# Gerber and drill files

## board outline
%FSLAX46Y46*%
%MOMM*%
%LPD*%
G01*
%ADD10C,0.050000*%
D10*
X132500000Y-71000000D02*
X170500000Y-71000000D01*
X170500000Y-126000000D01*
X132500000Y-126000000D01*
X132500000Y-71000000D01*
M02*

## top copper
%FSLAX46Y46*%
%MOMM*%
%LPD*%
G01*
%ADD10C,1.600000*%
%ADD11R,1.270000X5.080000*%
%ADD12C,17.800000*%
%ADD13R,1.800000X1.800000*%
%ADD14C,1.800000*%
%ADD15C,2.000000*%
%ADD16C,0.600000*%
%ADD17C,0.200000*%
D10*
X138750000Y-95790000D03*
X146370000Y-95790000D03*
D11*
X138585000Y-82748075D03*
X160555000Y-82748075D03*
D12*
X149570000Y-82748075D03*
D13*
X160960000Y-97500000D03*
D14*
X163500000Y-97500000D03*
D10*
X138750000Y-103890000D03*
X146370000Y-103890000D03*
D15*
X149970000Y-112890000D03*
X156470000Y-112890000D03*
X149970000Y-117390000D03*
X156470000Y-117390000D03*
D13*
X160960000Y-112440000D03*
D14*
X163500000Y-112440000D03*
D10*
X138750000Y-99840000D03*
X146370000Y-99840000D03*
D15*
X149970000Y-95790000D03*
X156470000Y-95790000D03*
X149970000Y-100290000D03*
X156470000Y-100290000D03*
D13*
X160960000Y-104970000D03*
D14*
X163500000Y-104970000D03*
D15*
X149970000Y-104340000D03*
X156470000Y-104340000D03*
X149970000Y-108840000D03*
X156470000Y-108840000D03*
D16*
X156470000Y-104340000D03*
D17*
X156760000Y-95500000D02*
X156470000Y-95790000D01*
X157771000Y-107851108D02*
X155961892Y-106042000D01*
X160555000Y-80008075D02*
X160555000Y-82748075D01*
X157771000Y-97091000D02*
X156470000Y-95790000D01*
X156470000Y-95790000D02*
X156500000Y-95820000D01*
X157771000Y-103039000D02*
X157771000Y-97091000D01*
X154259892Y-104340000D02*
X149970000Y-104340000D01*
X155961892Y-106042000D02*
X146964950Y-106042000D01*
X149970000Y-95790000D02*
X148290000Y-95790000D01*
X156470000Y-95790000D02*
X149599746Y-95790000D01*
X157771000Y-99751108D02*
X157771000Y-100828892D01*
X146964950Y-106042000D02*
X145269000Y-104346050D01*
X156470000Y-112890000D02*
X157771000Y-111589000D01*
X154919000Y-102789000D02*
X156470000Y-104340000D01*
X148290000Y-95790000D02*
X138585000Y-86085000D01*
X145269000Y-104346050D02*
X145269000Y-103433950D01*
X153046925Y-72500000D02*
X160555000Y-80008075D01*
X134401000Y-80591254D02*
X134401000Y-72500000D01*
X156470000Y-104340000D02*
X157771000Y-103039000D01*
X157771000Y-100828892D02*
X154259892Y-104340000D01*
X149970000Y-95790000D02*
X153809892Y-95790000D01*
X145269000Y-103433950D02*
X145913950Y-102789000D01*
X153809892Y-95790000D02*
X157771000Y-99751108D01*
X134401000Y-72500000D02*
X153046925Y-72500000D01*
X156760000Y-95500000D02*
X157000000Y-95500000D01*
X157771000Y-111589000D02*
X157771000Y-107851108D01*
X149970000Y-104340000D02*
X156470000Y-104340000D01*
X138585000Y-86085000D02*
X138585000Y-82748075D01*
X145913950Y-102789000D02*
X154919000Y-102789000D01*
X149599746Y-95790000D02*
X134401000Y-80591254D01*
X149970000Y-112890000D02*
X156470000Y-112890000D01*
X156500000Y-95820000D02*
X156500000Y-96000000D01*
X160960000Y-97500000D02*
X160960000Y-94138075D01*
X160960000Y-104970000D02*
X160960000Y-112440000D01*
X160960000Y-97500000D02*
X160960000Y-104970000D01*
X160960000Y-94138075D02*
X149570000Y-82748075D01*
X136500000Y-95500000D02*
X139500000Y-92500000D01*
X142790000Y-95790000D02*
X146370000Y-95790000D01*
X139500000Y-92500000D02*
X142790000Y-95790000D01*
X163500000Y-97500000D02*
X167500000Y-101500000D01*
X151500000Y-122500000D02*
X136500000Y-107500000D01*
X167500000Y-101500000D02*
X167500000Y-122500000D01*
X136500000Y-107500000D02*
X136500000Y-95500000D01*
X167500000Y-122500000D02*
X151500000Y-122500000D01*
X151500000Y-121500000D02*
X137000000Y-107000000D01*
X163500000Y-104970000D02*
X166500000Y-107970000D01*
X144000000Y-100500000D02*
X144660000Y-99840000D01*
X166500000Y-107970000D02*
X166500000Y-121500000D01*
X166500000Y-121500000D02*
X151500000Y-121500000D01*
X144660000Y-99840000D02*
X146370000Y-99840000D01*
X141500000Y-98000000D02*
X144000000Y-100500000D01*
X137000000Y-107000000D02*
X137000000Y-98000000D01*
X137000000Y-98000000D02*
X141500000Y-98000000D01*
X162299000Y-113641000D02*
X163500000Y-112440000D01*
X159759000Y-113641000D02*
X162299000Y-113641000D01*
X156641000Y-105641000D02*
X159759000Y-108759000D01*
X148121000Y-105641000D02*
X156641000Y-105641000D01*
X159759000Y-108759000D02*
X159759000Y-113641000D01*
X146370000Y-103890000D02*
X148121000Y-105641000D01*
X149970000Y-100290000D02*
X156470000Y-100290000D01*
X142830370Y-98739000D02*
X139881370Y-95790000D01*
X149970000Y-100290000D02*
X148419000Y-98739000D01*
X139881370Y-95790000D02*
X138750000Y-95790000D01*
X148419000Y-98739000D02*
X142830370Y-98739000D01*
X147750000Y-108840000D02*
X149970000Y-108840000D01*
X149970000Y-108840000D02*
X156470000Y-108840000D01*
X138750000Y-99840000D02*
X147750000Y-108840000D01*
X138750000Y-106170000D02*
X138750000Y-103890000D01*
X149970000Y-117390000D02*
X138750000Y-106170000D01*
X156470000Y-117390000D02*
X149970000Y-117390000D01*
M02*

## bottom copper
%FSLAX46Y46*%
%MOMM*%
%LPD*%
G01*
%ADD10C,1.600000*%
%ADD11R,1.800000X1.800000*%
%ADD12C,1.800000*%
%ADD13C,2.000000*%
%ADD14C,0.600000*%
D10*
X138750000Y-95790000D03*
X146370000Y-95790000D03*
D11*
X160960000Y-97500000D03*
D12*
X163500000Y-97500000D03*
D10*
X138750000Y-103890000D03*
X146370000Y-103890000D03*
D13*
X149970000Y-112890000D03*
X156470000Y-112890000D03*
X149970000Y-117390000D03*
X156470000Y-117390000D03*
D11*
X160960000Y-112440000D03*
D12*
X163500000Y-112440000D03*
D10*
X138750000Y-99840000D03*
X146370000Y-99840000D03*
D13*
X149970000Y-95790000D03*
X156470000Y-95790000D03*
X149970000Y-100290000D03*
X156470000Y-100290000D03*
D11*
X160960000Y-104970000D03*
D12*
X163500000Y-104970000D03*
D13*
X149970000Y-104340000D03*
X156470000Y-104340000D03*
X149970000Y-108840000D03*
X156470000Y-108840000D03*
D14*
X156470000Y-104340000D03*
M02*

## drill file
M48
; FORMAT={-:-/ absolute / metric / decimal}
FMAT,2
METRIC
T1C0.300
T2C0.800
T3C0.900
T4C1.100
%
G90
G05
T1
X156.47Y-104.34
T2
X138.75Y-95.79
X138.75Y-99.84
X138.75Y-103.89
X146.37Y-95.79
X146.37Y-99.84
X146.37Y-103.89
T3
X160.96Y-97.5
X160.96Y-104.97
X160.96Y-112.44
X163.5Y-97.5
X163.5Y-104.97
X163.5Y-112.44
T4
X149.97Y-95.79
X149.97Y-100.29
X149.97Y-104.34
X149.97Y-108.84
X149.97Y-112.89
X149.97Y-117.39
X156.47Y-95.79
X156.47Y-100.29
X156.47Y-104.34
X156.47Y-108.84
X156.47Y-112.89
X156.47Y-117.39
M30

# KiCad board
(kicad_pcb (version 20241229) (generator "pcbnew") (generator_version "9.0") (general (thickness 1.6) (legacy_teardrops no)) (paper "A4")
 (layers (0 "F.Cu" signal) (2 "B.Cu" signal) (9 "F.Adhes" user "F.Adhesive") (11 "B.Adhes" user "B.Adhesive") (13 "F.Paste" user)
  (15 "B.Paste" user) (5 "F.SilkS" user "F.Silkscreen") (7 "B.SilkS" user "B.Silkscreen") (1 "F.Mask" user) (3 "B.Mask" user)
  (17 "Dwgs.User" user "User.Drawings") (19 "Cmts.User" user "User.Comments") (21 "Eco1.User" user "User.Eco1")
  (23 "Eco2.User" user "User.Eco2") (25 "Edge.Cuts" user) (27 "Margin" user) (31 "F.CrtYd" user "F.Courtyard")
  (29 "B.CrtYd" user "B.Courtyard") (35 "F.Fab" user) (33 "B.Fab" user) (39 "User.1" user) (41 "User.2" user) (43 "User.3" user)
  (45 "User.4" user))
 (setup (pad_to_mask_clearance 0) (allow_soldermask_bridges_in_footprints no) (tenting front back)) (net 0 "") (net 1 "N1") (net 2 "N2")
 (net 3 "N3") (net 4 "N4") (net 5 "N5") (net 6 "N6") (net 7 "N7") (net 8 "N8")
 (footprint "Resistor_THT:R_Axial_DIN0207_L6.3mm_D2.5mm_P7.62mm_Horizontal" (layer "F.Cu") (at 138.75 95.79)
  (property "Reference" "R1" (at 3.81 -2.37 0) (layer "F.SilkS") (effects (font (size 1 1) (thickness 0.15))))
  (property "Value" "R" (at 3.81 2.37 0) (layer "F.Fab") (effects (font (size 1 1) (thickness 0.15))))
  (pad "1" thru_hole circle (at 0 0) (size 1.6 1.6) (drill 0.8) (layers "*.Cu" "*.Mask") (remove_unused_layers no) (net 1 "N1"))
  (pad "2" thru_hole circle (at 7.62 0) (size 1.6 1.6) (drill 0.8) (layers "*.Cu" "*.Mask") (remove_unused_layers no) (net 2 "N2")))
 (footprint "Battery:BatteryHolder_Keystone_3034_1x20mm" (layer "F.Cu") (at 149.57 82.748075)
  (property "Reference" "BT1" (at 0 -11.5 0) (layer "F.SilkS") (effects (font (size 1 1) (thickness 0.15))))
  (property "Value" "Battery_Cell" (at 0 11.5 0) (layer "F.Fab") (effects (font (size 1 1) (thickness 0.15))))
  (pad "1" smd rect (at -10.985 0) (size 1.27 5.08) (layers "F.Cu" "F.Mask" "F.Paste") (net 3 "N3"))
  (pad "1" smd rect (at 10.985 0) (size 1.27 5.08) (layers "F.Cu" "F.Mask" "F.Paste") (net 3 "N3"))
  (pad "2" smd circle (at 0 0) (size 17.8 17.8) (layers "F.Cu" "F.Mask") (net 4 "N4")))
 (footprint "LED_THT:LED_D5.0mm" (layer "F.Cu") (at 160.96 97.5)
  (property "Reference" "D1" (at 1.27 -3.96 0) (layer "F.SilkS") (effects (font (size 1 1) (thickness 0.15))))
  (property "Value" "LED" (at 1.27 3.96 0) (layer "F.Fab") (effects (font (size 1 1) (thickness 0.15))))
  (pad "1" thru_hole rect (at 0 0) (size 1.8 1.8) (drill 0.9) (layers "*.Cu" "*.Mask") (remove_unused_layers no) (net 4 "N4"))
  (pad "2" thru_hole circle (at 2.54 0) (size 1.8 1.8) (drill 0.9) (layers "*.Cu" "*.Mask") (remove_unused_layers no) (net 2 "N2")))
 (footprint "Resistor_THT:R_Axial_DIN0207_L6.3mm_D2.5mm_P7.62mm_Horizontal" (layer "F.Cu") (at 138.75 103.89)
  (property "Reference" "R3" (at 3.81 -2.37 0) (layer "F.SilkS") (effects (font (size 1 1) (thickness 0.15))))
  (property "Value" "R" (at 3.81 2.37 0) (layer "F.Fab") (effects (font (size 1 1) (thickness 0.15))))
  (pad "1" thru_hole circle (at 0 0) (size 1.6 1.6) (drill 0.8) (layers "*.Cu" "*.Mask") (remove_unused_layers no) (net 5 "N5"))
  (pad "2" thru_hole circle (at 7.62 0) (size 1.6 1.6) (drill 0.8) (layers "*.Cu" "*.Mask") (remove_unused_layers no) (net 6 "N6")))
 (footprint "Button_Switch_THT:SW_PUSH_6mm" (layer "F.Cu") (at 149.97 112.89)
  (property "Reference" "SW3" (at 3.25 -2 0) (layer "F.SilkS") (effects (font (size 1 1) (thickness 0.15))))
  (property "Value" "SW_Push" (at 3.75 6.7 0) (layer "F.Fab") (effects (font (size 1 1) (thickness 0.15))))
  (pad "1" thru_hole circle (at 0 0 90) (size 2 2) (drill 1.1) (layers "*.Cu" "*.Mask") (remove_unused_layers no) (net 3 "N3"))
  (pad "1" thru_hole circle (at 6.5 0 90) (size 2 2) (drill 1.1) (layers "*.Cu" "*.Mask") (remove_unused_layers no) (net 3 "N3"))
  (pad "2" thru_hole circle (at 0 4.5 90) (size 2 2) (drill 1.1) (layers "*.Cu" "*.Mask") (remove_unused_layers no) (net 5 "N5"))
  (pad "2" thru_hole circle (at 6.5 4.5 90) (size 2 2) (drill 1.1) (layers "*.Cu" "*.Mask") (remove_unused_layers no) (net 5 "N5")))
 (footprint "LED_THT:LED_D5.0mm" (layer "F.Cu") (at 160.96 112.44)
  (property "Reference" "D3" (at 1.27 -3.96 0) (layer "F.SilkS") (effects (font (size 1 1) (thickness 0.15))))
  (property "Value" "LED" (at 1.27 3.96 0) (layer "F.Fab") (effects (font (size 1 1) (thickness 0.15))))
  (pad "1" thru_hole rect (at 0 0) (size 1.8 1.8) (drill 0.9) (layers "*.Cu" "*.Mask") (remove_unused_layers no) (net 4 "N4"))
  (pad "2" thru_hole circle (at 2.54 0) (size 1.8 1.8) (drill 0.9) (layers "*.Cu" "*.Mask") (remove_unused_layers no) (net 6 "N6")))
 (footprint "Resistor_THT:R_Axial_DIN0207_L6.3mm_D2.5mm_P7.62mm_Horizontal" (layer "F.Cu") (at 138.75 99.84)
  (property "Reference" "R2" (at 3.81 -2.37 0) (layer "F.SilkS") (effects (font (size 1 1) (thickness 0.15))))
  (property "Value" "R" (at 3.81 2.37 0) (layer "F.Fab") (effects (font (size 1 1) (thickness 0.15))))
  (pad "1" thru_hole circle (at 0 0) (size 1.6 1.6) (drill 0.8) (layers "*.Cu" "*.Mask") (remove_unused_layers no) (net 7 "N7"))
  (pad "2" thru_hole circle (at 7.62 0) (size 1.6 1.6) (drill 0.8) (layers "*.Cu" "*.Mask") (remove_unused_layers no) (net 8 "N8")))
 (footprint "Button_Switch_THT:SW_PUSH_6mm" (layer "F.Cu") (at 149.97 95.79)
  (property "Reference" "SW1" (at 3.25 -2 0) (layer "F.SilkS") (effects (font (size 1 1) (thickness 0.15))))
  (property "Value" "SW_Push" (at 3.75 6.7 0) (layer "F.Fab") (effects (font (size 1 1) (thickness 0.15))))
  (pad "1" thru_hole circle (at 0 0 90) (size 2 2) (drill 1.1) (layers "*.Cu" "*.Mask") (remove_unused_layers no) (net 3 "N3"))
  (pad "1" thru_hole circle (at 6.5 0 90) (size 2 2) (drill 1.1) (layers "*.Cu" "*.Mask") (remove_unused_layers no) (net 3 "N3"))
  (pad "2" thru_hole circle (at 0 4.5 90) (size 2 2) (drill 1.1) (layers "*.Cu" "*.Mask") (remove_unused_layers no) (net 1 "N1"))
  (pad "2" thru_hole circle (at 6.5 4.5 90) (size 2 2) (drill 1.1) (layers "*.Cu" "*.Mask") (remove_unused_layers no) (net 1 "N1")))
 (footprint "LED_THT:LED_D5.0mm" (layer "F.Cu") (at 160.96 104.97)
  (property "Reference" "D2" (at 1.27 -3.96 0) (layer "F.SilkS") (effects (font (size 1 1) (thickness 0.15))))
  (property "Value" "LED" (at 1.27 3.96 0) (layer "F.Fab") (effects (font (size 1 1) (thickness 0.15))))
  (pad "1" thru_hole rect (at 0 0) (size 1.8 1.8) (drill 0.9) (layers "*.Cu" "*.Mask") (remove_unused_layers no) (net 4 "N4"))
  (pad "2" thru_hole circle (at 2.54 0) (size 1.8 1.8) (drill 0.9) (layers "*.Cu" "*.Mask") (remove_unused_layers no) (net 8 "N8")))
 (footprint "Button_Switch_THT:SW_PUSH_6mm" (layer "F.Cu") (at 149.97 104.34)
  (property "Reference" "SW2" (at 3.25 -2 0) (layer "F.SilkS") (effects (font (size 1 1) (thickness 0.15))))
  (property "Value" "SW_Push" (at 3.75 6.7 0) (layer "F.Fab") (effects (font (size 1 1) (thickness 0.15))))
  (pad "1" thru_hole circle (at 0 0 90) (size 2 2) (drill 1.1) (layers "*.Cu" "*.Mask") (remove_unused_layers no) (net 3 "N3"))
  (pad "1" thru_hole circle (at 6.5 0 90) (size 2 2) (drill 1.1) (layers "*.Cu" "*.Mask") (remove_unused_layers no) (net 3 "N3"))
  (pad "2" thru_hole circle (at 0 4.5 90) (size 2 2) (drill 1.1) (layers "*.Cu" "*.Mask") (remove_unused_layers no) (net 7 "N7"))
  (pad "2" thru_hole circle (at 6.5 4.5 90) (size 2 2) (drill 1.1) (layers "*.Cu" "*.Mask") (remove_unused_layers no) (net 7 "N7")))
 (gr_rect (start 132.5 71) (end 170.5 126) (stroke (width 0.05) (type default)) (fill no) (layer "Edge.Cuts"))
 (segment (start 156.76 95.5) (end 156.47 95.79) (width 0.2) (layer "F.Cu") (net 3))
 (segment (start 157.771 107.851108) (end 155.961892 106.042) (width 0.2) (layer "F.Cu") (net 3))
 (segment (start 160.555 80.008075) (end 160.555 82.748075) (width 0.2) (layer "F.Cu") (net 3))
 (segment (start 157.771 97.091) (end 156.47 95.79) (width 0.2) (layer "F.Cu") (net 3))
 (segment (start 156.47 95.79) (end 156.5 95.82) (width 0.2) (layer "F.Cu") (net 3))
 (segment (start 157.771 103.039) (end 157.771 97.091) (width 0.2) (layer "F.Cu") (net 3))
 (segment (start 154.259892 104.34) (end 149.97 104.34) (width 0.2) (layer "F.Cu") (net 3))
 (segment (start 155.961892 106.042) (end 146.96495 106.042) (width 0.2) (layer "F.Cu") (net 3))
 (segment (start 149.97 95.79) (end 148.29 95.79) (width 0.2) (layer "F.Cu") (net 3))
 (segment (start 156.47 95.79) (end 149.599746 95.79) (width 0.2) (layer "F.Cu") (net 3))
 (segment (start 157.771 99.751108) (end 157.771 100.828892) (width 0.2) (layer "F.Cu") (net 3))
 (segment (start 146.96495 106.042) (end 145.269 104.34605) (width 0.2) (layer "F.Cu") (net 3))
 (segment (start 156.47 112.89) (end 157.771 111.589) (width 0.2) (layer "F.Cu") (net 3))
 (segment (start 154.919 102.789) (end 156.47 104.34) (width 0.2) (layer "F.Cu") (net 3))
 (segment (start 148.29 95.79) (end 138.585 86.085) (width 0.2) (layer "F.Cu") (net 3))
 (segment (start 145.269 104.34605) (end 145.269 103.43395) (width 0.2) (layer "F.Cu") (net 3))
 (segment (start 153.046925 72.5) (end 160.555 80.008075) (width 0.2) (layer "F.Cu") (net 3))
 (segment (start 134.401 80.591254) (end 134.401 72.5) (width 0.2) (layer "F.Cu") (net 3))
 (segment (start 156.47 104.34) (end 157.771 103.039) (width 0.2) (layer "F.Cu") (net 3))
 (segment (start 157.771 100.828892) (end 154.259892 104.34) (width 0.2) (layer "F.Cu") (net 3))
 (segment (start 149.97 95.79) (end 153.809892 95.79) (width 0.2) (layer "F.Cu") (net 3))
 (segment (start 145.269 103.43395) (end 145.91395 102.789) (width 0.2) (layer "F.Cu") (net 3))
 (segment (start 153.809892 95.79) (end 157.771 99.751108) (width 0.2) (layer "F.Cu") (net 3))
 (segment (start 134.401 72.5) (end 153.046925 72.5) (width 0.2) (layer "F.Cu") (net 3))
 (segment (start 156.76 95.5) (end 157 95.5) (width 0.2) (layer "F.Cu") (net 3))
 (segment (start 157.771 111.589) (end 157.771 107.851108) (width 0.2) (layer "F.Cu") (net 3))
 (segment (start 149.97 104.34) (end 156.47 104.34) (width 0.2) (layer "F.Cu") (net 3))
 (segment (start 138.585 86.085) (end 138.585 82.748075) (width 0.2) (layer "F.Cu") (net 3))
 (segment (start 145.91395 102.789) (end 154.919 102.789) (width 0.2) (layer "F.Cu") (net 3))
 (segment (start 149.599746 95.79) (end 134.401 80.591254) (width 0.2) (layer "F.Cu") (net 3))
 (segment (start 149.97 112.89) (end 156.47 112.89) (width 0.2) (layer "F.Cu") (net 3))
 (segment (start 156.5 95.82) (end 156.5 96) (width 0.2) (layer "F.Cu") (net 3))
 (via (at 156.47 104.34) (size 0.6) (drill 0.3) (layers "F.Cu" "B.Cu") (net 3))
 (segment (start 160.96 97.5) (end 160.96 94.138075) (width 0.2) (layer "F.Cu") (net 4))
 (segment (start 160.96 104.97) (end 160.96 112.44) (width 0.2) (layer "F.Cu") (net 4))
 (segment (start 160.96 97.5) (end 160.96 104.97) (width 0.2) (layer "F.Cu") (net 4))
 (segment (start 160.96 94.138075) (end 149.57 82.748075) (width 0.2) (layer "F.Cu") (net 4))
 (segment (start 136.5 95.5) (end 139.5 92.5) (width 0.2) (layer "F.Cu") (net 2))
 (segment (start 142.79 95.79) (end 146.37 95.79) (width 0.2) (layer "F.Cu") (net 2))
 (segment (start 139.5 92.5) (end 142.79 95.79) (width 0.2) (layer "F.Cu") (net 2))
 (segment (start 163.5 97.5) (end 167.5 101.5) (width 0.2) (layer "F.Cu") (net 2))
 (segment (start 151.5 122.5) (end 136.5 107.5) (width 0.2) (layer "F.Cu") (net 2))
 (segment (start 167.5 101.5) (end 167.5 122.5) (width 0.2) (layer "F.Cu") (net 2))
 (segment (start 136.5 107.5) (end 136.5 95.5) (width 0.2) (layer "F.Cu") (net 2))
 (segment (start 167.5 122.5) (end 151.5 122.5) (width 0.2) (layer "F.Cu") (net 2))
 (segment (start 151.5 121.5) (end 137 107) (width 0.2) (layer "F.Cu") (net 8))
 (segment (start 163.5 104.97) (end 166.5 107.97) (width 0.2) (layer "F.Cu") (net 8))
 (segment (start 144 100.5) (end 144.66 99.84) (width 0.2) (layer "F.Cu") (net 8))
 (segment (start 166.5 107.97) (end 166.5 121.5) (width 0.2) (layer "F.Cu") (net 8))
 (segment (start 166.5 121.5) (end 151.5 121.5) (width 0.2) (layer "F.Cu") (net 8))
 (segment (start 144.66 99.84) (end 146.37 99.84) (width 0.2) (layer "F.Cu") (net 8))
 (segment (start 141.5 98) (end 144 100.5) (width 0.2) (layer "F.Cu") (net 8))
 (segment (start 137 107) (end 137 98) (width 0.2) (layer "F.Cu") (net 8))
 (segment (start 137 98) (end 141.5 98) (width 0.2) (layer "F.Cu") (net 8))
 (segment (start 162.299 113.641) (end 163.5 112.44) (width 0.2) (layer "F.Cu") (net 6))
 (segment (start 159.759 113.641) (end 162.299 113.641) (width 0.2) (layer "F.Cu") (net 6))
 (segment (start 156.641 105.641) (end 159.759 108.759) (width 0.2) (layer "F.Cu") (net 6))
 (segment (start 148.121 105.641) (end 156.641 105.641) (width 0.2) (layer "F.Cu") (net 6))
 (segment (start 159.759 108.759) (end 159.759 113.641) (width 0.2) (layer "F.Cu") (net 6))
 (segment (start 146.37 103.89) (end 148.121 105.641) (width 0.2) (layer "F.Cu") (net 6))
 (segment (start 149.97 100.29) (end 156.47 100.29) (width 0.2) (layer "F.Cu") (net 1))
 (segment (start 142.83037 98.739) (end 139.88137 95.79) (width 0.2) (layer "F.Cu") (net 1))
 (segment (start 149.97 100.29) (end 148.419 98.739) (width 0.2) (layer "F.Cu") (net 1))
 (segment (start 139.88137 95.79) (end 138.75 95.79) (width 0.2) (layer "F.Cu") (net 1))
 (segment (start 148.419 98.739) (end 142.83037 98.739) (width 0.2) (layer "F.Cu") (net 1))
 (segment (start 147.75 108.84) (end 149.97 108.84) (width 0.2) (layer "F.Cu") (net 7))
 (segment (start 149.97 108.84) (end 156.47 108.84) (width 0.2) (layer "F.Cu") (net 7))
 (segment (start 138.75 99.84) (end 147.75 108.84) (width 0.2) (layer "F.Cu") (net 7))
 (segment (start 138.75 106.17) (end 138.75 103.89) (width 0.2) (layer "F.Cu") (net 5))
 (segment (start 149.97 117.39) (end 138.75 106.17) (width 0.2) (layer "F.Cu") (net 5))
 (segment (start 156.47 117.39) (end 149.97 117.39) (width 0.2) (layer "F.Cu") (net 5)))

